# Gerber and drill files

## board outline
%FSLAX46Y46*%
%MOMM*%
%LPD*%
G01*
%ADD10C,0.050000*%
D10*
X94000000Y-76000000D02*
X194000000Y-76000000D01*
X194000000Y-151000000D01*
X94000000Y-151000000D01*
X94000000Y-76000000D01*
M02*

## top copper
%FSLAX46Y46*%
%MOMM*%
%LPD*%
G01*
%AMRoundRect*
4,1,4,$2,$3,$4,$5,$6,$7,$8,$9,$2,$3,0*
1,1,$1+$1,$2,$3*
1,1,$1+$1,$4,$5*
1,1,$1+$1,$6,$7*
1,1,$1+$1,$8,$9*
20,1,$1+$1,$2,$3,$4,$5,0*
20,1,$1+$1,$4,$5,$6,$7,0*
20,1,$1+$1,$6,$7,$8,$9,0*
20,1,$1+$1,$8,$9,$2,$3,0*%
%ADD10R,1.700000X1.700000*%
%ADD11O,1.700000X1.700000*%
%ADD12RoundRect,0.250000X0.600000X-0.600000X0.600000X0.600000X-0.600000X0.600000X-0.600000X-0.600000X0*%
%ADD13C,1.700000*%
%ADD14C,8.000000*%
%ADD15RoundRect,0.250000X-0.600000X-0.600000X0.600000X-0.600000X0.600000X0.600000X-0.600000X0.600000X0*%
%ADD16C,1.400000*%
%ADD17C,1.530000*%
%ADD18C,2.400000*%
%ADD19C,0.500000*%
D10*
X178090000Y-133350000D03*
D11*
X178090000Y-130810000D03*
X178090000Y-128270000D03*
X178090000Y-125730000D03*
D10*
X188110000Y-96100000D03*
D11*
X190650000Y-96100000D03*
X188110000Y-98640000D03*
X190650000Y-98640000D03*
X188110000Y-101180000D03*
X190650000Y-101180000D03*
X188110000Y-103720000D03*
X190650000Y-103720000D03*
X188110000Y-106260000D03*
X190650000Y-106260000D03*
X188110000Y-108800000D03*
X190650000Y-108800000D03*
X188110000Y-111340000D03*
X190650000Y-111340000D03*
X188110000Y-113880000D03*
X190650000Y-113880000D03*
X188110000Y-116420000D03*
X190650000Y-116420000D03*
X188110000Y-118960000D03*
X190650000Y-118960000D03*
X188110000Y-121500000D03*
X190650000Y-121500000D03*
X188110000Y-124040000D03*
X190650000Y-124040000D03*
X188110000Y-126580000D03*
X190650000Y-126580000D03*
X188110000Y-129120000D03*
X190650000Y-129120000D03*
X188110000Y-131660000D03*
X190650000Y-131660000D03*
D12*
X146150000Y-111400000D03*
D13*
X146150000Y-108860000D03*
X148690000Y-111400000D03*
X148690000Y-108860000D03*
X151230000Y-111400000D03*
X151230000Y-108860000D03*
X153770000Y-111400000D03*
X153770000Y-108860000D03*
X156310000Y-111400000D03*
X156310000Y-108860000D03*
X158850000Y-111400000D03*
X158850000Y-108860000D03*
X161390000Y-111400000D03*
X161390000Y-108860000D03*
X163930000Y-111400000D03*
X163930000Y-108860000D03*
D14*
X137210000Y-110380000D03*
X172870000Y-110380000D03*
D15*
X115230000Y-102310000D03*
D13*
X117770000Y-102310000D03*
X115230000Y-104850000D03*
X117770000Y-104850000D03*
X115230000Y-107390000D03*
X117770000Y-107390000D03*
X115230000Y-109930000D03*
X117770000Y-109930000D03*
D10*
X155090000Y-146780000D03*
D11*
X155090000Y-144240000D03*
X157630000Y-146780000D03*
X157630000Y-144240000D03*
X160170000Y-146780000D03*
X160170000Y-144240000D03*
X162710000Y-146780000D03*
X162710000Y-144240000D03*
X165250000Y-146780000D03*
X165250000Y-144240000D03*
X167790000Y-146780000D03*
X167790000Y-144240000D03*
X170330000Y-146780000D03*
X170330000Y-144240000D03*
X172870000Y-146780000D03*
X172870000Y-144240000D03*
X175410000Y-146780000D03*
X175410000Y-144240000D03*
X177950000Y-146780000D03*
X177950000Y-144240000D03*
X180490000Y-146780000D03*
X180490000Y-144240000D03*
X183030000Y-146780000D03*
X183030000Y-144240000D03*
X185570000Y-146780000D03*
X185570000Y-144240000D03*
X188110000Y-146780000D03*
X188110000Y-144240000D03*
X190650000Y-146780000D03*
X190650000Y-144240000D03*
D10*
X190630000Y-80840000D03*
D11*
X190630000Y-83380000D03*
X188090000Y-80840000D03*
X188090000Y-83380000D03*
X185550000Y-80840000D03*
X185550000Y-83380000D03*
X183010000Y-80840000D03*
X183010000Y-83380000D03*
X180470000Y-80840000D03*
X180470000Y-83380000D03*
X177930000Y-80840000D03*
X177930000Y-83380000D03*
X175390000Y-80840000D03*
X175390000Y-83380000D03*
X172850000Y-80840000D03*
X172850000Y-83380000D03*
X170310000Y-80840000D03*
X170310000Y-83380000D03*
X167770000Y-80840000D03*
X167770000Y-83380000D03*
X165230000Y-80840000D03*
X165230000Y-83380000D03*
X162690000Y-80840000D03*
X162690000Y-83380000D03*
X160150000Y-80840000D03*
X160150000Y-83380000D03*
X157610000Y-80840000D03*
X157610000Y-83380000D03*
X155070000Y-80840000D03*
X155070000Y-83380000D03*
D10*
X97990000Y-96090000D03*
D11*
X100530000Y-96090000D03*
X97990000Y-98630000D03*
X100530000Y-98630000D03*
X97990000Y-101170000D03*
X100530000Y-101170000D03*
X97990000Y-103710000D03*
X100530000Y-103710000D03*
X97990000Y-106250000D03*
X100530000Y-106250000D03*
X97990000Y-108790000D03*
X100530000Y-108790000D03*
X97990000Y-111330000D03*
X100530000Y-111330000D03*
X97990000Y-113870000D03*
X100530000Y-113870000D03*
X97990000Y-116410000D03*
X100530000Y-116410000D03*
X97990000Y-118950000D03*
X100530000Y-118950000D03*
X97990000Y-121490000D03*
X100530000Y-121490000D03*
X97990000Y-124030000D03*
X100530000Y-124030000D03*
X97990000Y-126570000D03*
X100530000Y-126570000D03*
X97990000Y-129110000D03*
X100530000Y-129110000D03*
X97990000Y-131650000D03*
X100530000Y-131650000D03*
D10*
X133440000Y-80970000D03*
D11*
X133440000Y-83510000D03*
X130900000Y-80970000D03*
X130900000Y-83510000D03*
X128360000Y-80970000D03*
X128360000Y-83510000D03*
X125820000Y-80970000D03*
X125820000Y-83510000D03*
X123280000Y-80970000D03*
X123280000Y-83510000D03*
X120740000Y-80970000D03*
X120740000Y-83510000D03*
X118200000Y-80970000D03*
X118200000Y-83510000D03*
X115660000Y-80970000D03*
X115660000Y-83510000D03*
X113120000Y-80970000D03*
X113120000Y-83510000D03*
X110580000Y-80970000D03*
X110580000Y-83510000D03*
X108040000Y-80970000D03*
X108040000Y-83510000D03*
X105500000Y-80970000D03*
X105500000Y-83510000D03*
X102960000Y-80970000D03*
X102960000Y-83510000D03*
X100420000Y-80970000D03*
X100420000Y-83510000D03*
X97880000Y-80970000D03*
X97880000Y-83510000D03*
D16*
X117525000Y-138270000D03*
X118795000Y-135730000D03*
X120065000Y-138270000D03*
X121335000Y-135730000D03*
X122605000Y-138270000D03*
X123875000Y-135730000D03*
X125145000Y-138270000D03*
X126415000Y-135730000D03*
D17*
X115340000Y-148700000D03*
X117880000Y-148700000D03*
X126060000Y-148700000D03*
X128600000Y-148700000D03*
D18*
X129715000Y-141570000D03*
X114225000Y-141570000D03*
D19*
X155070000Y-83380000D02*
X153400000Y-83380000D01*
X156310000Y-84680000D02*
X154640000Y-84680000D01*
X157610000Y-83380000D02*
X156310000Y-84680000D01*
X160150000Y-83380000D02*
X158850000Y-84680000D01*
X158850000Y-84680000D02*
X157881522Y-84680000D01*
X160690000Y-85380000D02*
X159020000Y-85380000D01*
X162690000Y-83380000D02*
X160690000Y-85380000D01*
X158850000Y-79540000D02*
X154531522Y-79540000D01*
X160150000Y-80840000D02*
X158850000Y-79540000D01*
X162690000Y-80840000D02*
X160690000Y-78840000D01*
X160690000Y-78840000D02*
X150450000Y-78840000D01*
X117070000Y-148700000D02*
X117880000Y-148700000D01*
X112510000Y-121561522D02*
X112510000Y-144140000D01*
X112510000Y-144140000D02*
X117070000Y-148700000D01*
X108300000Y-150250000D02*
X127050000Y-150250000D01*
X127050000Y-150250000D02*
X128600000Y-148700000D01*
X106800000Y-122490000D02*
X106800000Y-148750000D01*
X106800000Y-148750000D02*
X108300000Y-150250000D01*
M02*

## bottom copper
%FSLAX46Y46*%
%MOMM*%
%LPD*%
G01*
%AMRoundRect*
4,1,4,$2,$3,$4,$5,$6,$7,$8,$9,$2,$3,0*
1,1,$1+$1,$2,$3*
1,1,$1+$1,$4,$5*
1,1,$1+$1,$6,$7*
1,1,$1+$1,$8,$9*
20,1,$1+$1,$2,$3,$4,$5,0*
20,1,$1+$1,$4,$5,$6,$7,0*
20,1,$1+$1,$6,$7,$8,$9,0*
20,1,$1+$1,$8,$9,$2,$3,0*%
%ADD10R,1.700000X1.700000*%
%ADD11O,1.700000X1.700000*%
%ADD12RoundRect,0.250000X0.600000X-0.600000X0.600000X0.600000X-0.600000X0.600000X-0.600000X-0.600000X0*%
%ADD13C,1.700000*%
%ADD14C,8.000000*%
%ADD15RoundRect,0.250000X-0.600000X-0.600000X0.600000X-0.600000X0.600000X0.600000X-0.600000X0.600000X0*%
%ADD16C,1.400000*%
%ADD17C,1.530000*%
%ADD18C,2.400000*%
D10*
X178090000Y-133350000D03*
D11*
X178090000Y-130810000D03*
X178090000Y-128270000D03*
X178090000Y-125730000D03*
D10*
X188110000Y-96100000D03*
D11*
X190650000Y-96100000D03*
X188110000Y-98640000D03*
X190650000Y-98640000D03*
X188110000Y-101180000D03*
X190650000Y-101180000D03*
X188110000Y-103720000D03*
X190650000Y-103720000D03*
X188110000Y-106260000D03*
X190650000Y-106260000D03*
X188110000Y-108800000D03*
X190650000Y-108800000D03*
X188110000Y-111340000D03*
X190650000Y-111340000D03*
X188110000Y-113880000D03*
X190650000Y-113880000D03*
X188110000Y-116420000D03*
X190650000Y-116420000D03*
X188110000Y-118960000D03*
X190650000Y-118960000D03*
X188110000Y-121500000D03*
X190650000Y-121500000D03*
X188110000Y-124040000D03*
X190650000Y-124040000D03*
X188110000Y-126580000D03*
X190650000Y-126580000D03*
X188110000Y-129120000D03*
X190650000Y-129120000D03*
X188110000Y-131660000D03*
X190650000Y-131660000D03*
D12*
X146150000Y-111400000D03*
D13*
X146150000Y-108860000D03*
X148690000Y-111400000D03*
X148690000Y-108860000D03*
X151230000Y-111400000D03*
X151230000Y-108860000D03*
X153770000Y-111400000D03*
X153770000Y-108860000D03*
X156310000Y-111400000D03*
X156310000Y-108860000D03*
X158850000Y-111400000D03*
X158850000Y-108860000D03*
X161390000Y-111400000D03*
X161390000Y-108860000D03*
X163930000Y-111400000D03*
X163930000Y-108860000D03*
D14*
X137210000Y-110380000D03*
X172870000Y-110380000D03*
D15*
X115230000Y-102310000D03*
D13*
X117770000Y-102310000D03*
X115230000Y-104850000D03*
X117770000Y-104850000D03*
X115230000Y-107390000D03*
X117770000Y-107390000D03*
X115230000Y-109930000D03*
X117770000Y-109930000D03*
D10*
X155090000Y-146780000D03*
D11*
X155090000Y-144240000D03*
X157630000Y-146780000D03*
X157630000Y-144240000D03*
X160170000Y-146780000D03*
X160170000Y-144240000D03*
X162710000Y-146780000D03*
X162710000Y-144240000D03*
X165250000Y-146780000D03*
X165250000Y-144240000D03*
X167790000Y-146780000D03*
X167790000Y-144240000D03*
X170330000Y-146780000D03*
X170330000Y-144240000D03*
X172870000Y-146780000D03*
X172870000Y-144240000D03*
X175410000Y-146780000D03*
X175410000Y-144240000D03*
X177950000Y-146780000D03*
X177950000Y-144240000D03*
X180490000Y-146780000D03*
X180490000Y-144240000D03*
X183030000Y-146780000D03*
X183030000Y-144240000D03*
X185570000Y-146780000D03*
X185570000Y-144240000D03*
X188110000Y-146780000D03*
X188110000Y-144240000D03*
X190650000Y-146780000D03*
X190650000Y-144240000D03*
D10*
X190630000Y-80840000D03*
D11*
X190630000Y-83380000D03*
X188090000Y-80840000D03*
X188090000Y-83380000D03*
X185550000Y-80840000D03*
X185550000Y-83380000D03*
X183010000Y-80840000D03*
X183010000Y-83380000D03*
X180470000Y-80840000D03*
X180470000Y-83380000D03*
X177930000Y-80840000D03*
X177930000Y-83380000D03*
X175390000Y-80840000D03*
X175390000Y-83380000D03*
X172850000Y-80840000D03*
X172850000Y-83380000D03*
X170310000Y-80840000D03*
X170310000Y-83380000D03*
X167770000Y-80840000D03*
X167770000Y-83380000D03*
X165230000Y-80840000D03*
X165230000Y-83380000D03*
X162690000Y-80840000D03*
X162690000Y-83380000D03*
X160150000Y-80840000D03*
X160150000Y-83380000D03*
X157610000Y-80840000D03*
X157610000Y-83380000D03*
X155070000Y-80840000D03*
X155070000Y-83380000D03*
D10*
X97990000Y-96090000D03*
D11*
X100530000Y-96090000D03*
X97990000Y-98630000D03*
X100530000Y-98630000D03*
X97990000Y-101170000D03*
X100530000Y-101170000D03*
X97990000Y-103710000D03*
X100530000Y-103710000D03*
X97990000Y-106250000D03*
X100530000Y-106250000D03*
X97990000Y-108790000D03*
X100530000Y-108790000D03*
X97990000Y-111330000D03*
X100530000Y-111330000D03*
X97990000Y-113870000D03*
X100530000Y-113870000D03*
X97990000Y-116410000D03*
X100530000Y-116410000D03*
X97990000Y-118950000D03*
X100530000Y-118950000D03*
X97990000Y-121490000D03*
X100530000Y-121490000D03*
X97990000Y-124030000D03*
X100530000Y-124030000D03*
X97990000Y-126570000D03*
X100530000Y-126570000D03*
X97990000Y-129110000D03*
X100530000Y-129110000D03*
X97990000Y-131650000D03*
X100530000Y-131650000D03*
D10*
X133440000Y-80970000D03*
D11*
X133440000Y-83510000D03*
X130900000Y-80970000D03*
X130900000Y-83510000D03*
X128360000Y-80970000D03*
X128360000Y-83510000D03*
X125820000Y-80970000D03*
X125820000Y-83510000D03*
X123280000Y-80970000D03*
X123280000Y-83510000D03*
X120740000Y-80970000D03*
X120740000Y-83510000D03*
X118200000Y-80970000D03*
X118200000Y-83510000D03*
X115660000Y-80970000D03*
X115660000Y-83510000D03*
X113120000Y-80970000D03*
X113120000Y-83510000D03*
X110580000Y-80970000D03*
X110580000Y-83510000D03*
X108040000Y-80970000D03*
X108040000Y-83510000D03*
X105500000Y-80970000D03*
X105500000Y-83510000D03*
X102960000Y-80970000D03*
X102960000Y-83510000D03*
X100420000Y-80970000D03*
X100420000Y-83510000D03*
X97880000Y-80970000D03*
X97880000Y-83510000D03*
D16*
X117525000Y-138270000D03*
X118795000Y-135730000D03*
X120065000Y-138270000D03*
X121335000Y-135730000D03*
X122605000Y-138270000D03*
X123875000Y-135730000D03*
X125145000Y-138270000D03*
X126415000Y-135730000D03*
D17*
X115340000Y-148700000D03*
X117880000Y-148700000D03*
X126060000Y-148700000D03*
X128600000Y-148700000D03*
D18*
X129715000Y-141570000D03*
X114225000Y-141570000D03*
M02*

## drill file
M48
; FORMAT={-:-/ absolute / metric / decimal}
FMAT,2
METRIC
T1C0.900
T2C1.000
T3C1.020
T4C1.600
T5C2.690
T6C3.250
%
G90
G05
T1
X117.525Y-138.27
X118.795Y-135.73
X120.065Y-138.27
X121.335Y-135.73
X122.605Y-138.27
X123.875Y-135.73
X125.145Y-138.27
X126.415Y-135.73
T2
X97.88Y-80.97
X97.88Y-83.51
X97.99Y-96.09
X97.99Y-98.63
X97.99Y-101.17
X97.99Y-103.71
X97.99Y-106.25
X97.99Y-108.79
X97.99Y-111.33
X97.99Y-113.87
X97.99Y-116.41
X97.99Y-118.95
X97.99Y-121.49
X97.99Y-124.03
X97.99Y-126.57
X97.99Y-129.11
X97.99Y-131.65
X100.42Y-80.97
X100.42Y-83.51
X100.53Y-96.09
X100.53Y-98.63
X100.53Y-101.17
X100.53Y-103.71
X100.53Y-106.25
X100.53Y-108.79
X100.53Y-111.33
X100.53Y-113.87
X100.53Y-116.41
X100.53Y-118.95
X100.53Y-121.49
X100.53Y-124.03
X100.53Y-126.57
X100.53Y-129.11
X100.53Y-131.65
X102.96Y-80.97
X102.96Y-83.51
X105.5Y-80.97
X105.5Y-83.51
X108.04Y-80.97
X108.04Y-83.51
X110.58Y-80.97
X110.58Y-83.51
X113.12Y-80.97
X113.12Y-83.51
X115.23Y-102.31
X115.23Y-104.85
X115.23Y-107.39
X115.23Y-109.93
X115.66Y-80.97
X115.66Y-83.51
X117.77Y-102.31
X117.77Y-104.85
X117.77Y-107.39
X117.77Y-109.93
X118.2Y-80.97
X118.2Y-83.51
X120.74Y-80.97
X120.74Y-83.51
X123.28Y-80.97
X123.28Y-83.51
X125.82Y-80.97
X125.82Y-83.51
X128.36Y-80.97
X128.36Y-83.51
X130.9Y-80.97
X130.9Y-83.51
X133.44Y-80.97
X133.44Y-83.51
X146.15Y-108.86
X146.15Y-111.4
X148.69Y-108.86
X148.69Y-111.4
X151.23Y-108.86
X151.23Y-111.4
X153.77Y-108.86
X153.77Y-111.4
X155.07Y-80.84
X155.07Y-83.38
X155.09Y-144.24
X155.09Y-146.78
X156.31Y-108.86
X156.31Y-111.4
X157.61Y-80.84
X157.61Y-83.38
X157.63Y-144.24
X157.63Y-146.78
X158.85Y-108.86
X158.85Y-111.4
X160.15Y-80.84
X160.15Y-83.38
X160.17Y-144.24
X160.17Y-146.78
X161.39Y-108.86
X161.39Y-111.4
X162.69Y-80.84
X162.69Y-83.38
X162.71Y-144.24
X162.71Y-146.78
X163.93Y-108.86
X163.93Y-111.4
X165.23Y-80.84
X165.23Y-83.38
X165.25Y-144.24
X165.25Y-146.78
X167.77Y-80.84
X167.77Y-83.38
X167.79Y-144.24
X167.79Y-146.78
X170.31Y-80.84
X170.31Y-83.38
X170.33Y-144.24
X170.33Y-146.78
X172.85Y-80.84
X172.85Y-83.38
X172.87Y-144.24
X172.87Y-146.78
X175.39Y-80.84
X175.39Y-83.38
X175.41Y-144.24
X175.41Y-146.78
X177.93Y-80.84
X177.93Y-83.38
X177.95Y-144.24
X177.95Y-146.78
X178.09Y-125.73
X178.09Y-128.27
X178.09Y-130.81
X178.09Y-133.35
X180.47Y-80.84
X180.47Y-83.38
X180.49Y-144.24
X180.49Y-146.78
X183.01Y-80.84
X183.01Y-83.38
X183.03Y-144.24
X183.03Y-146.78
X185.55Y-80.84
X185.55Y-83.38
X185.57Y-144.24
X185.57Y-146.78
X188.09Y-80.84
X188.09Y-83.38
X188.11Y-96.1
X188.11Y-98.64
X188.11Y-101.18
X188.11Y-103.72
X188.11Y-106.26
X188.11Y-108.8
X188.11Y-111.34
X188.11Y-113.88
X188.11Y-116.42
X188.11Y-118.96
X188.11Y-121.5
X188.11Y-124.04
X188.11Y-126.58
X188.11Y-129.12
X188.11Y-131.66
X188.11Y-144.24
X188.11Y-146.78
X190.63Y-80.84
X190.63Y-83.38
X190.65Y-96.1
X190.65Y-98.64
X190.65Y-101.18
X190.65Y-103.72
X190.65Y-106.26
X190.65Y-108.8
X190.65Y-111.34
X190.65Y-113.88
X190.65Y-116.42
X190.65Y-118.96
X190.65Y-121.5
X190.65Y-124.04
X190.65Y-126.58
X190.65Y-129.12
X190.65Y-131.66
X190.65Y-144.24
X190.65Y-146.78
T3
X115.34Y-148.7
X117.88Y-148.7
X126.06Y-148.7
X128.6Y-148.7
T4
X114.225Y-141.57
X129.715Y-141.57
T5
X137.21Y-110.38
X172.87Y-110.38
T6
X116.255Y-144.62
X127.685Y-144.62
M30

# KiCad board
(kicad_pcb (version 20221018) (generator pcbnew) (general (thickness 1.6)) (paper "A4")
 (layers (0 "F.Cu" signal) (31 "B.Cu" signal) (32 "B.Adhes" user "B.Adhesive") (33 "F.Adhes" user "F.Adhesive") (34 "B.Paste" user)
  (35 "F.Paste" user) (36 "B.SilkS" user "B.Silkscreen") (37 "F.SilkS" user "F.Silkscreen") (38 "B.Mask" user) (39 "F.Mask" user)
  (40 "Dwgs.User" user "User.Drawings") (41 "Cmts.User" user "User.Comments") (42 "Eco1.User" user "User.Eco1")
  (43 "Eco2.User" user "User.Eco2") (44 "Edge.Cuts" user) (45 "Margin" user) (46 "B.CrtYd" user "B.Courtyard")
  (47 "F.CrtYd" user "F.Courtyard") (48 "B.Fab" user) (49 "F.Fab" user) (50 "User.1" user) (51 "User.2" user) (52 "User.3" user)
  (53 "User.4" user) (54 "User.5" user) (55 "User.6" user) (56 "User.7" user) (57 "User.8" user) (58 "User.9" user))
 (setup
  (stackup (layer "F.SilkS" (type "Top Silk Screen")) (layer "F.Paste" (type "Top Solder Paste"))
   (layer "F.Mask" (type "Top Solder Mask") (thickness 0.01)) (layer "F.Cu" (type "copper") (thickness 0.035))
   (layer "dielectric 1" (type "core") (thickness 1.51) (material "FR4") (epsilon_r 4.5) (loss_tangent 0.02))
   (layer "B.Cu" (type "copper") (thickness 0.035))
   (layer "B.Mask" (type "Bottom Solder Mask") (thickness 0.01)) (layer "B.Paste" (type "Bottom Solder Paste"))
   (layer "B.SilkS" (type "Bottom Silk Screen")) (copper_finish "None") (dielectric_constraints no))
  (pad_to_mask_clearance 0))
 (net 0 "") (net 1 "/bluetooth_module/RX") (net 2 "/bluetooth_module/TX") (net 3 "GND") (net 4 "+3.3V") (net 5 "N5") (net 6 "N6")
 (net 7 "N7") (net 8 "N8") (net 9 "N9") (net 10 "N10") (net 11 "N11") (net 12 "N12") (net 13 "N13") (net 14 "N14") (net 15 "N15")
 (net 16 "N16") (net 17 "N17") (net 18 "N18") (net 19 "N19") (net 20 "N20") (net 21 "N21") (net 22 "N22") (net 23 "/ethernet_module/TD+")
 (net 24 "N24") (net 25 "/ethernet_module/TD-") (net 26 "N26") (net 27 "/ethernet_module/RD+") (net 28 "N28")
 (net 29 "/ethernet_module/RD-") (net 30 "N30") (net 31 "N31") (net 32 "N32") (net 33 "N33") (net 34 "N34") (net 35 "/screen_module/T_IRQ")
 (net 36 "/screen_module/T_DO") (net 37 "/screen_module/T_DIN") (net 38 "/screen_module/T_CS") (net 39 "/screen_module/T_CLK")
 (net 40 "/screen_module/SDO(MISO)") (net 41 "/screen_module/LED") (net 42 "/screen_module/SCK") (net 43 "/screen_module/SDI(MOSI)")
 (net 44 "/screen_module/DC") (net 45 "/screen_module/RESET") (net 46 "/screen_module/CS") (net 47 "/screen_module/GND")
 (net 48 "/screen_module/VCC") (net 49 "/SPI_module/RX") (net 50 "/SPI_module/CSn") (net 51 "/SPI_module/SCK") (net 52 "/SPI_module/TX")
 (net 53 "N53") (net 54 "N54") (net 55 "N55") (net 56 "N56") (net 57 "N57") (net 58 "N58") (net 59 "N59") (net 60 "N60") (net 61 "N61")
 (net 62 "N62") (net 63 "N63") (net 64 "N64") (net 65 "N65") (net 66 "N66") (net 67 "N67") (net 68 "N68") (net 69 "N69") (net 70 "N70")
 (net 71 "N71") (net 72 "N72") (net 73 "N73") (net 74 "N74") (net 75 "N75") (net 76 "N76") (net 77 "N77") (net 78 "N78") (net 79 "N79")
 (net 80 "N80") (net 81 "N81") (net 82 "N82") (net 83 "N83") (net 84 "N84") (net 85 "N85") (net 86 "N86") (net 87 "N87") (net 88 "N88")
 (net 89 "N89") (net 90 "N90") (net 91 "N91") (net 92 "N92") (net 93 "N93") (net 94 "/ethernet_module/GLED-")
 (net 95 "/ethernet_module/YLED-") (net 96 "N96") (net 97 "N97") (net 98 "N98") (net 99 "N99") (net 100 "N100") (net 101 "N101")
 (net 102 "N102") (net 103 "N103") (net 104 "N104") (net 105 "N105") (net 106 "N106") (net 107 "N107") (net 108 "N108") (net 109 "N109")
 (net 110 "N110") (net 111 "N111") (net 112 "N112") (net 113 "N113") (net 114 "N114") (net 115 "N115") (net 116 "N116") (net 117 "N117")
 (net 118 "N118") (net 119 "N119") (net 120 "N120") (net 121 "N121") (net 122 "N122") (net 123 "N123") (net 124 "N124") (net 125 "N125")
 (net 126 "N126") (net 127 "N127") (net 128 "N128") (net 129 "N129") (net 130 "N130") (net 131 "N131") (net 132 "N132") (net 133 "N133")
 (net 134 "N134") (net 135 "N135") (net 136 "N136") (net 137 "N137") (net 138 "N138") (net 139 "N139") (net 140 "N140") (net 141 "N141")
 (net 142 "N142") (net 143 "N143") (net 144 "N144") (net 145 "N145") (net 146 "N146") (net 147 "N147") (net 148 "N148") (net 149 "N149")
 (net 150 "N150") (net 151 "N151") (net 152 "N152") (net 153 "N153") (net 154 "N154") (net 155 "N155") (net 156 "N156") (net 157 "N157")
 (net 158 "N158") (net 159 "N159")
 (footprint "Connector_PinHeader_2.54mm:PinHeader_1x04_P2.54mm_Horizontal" (layer "F.Cu") (at 178.09 133.35 180)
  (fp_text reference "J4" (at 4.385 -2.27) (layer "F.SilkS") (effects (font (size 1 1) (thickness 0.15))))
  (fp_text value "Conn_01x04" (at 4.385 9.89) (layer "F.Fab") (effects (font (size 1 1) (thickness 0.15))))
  (pad "1" thru_hole rect (at 0 0 180) (size 1.7 1.7) (drill 1) (layers "*.Cu" "*.Mask") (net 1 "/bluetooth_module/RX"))
  (pad "2" thru_hole oval (at 0 2.54 180) (size 1.7 1.7) (drill 1) (layers "*.Cu" "*.Mask") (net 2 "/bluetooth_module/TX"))
  (pad "3" thru_hole oval (at 0 5.08 180) (size 1.7 1.7) (drill 1) (layers "*.Cu" "*.Mask") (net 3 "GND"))
  (pad "4" thru_hole oval (at 0 7.62 180) (size 1.7 1.7) (drill 1) (layers "*.Cu" "*.Mask") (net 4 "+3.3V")))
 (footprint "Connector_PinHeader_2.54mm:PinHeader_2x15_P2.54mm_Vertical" (layer "F.Cu") (at 188.11 96.1)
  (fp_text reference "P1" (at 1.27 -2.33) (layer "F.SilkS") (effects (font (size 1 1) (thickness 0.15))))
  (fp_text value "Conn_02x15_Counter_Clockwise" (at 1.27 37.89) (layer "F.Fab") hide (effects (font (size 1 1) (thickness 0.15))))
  (pad "1" thru_hole rect (at 0 0) (size 1.7 1.7) (drill 1) (layers "*.Cu" "*.Mask") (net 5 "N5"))
  (pad "2" thru_hole oval (at 2.54 0) (size 1.7 1.7) (drill 1) (layers "*.Cu" "*.Mask") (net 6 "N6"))
  (pad "3" thru_hole oval (at 0 2.54) (size 1.7 1.7) (drill 1) (layers "*.Cu" "*.Mask") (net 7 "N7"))
  (pad "4" thru_hole oval (at 2.54 2.54) (size 1.7 1.7) (drill 1) (layers "*.Cu" "*.Mask") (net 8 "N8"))
  (pad "5" thru_hole oval (at 0 5.08) (size 1.7 1.7) (drill 1) (layers "*.Cu" "*.Mask") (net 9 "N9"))
  (pad "6" thru_hole oval (at 2.54 5.08) (size 1.7 1.7) (drill 1) (layers "*.Cu" "*.Mask") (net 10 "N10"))
  (pad "7" thru_hole oval (at 0 7.62) (size 1.7 1.7) (drill 1) (layers "*.Cu" "*.Mask") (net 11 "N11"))
  (pad "8" thru_hole oval (at 2.54 7.62) (size 1.7 1.7) (drill 1) (layers "*.Cu" "*.Mask") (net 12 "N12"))
  (pad "9" thru_hole oval (at 0 10.16) (size 1.7 1.7) (drill 1) (layers "*.Cu" "*.Mask") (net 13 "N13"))
  (pad "10" thru_hole oval (at 2.54 10.16) (size 1.7 1.7) (drill 1) (layers "*.Cu" "*.Mask") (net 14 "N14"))
  (pad "11" thru_hole oval (at 0 12.7) (size 1.7 1.7) (drill 1) (layers "*.Cu" "*.Mask") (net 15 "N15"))
  (pad "12" thru_hole oval (at 2.54 12.7) (size 1.7 1.7) (drill 1) (layers "*.Cu" "*.Mask") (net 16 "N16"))
  (pad "13" thru_hole oval (at 0 15.24) (size 1.7 1.7) (drill 1) (layers "*.Cu" "*.Mask") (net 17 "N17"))
  (pad "14" thru_hole oval (at 2.54 15.24) (size 1.7 1.7) (drill 1) (layers "*.Cu" "*.Mask") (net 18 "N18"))
  (pad "15" thru_hole oval (at 0 17.78) (size 1.7 1.7) (drill 1) (layers "*.Cu" "*.Mask") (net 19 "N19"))
  (pad "16" thru_hole oval (at 2.54 17.78) (size 1.7 1.7) (drill 1) (layers "*.Cu" "*.Mask") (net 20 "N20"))
  (pad "17" thru_hole oval (at 0 20.32) (size 1.7 1.7) (drill 1) (layers "*.Cu" "*.Mask") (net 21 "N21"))
  (pad "18" thru_hole oval (at 2.54 20.32) (size 1.7 1.7) (drill 1) (layers "*.Cu" "*.Mask") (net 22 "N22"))
  (pad "19" thru_hole oval (at 0 22.86) (size 1.7 1.7) (drill 1) (layers "*.Cu" "*.Mask") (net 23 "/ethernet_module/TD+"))
  (pad "20" thru_hole oval (at 2.54 22.86) (size 1.7 1.7) (drill 1) (layers "*.Cu" "*.Mask") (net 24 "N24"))
  (pad "21" thru_hole oval (at 0 25.4) (size 1.7 1.7) (drill 1) (layers "*.Cu" "*.Mask") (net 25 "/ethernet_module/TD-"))
  (pad "22" thru_hole oval (at 2.54 25.4) (size 1.7 1.7) (drill 1) (layers "*.Cu" "*.Mask") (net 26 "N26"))
  (pad "23" thru_hole oval (at 0 27.94) (size 1.7 1.7) (drill 1) (layers "*.Cu" "*.Mask") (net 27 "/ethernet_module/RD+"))
  (pad "24" thru_hole oval (at 2.54 27.94) (size 1.7 1.7) (drill 1) (layers "*.Cu" "*.Mask") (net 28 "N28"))
  (pad "25" thru_hole oval (at 0 30.48) (size 1.7 1.7) (drill 1) (layers "*.Cu" "*.Mask") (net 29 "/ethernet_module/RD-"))
  (pad "26" thru_hole oval (at 2.54 30.48) (size 1.7 1.7) (drill 1) (layers "*.Cu" "*.Mask") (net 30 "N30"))
  (pad "27" thru_hole oval (at 0 33.02) (size 1.7 1.7) (drill 1) (layers "*.Cu" "*.Mask") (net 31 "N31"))
  (pad "28" thru_hole oval (at 2.54 33.02) (size 1.7 1.7) (drill 1) (layers "*.Cu" "*.Mask") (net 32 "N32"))
  (pad "29" thru_hole oval (at 0 35.56) (size 1.7 1.7) (drill 1) (layers "*.Cu" "*.Mask") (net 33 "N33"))
  (pad "30" thru_hole oval (at 2.54 35.56) (size 1.7 1.7) (drill 1) (layers "*.Cu" "*.Mask") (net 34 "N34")))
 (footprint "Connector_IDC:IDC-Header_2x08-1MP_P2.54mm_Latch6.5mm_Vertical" (layer "F.Cu") (at 146.15 111.4 90)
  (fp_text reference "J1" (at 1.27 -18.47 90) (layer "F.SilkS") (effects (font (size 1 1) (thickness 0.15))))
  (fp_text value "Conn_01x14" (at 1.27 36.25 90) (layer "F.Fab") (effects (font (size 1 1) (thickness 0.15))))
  (pad "1" thru_hole roundrect (at 0 0 90) (size 1.7 1.7) (drill 1) (layers "*.Cu" "*.Mask") (roundrect_rratio 0.147059)
   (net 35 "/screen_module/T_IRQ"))
  (pad "2" thru_hole circle (at 2.54 0 90) (size 1.7 1.7) (drill 1) (layers "*.Cu" "*.Mask") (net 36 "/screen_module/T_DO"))
  (pad "3" thru_hole circle (at 0 2.54 90) (size 1.7 1.7) (drill 1) (layers "*.Cu" "*.Mask") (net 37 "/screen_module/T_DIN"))
  (pad "4" thru_hole circle (at 2.54 2.54 90) (size 1.7 1.7) (drill 1) (layers "*.Cu" "*.Mask") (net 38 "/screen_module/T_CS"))
  (pad "5" thru_hole circle (at 0 5.08 90) (size 1.7 1.7) (drill 1) (layers "*.Cu" "*.Mask") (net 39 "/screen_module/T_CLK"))
  (pad "6" thru_hole circle (at 2.54 5.08 90) (size 1.7 1.7) (drill 1) (layers "*.Cu" "*.Mask") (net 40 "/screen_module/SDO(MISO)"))
  (pad "7" thru_hole circle (at 0 7.62 90) (size 1.7 1.7) (drill 1) (layers "*.Cu" "*.Mask") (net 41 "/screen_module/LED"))
  (pad "8" thru_hole circle (at 2.54 7.62 90) (size 1.7 1.7) (drill 1) (layers "*.Cu" "*.Mask") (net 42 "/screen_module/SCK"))
  (pad "9" thru_hole circle (at 0 10.16 90) (size 1.7 1.7) (drill 1) (layers "*.Cu" "*.Mask") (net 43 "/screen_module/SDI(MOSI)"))
  (pad "10" thru_hole circle (at 2.54 10.16 90) (size 1.7 1.7) (drill 1) (layers "*.Cu" "*.Mask") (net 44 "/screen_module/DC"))
  (pad "11" thru_hole circle (at 0 12.7 90) (size 1.7 1.7) (drill 1) (layers "*.Cu" "*.Mask") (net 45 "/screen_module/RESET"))
  (pad "12" thru_hole circle (at 2.54 12.7 90) (size 1.7 1.7) (drill 1) (layers "*.Cu" "*.Mask") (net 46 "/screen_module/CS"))
  (pad "13" thru_hole circle (at 0 15.24 90) (size 1.7 1.7) (drill 1) (layers "*.Cu" "*.Mask") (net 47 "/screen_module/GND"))
  (pad "14" thru_hole circle (at 2.54 15.24 90) (size 1.7 1.7) (drill 1) (layers "*.Cu" "*.Mask") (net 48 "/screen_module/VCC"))
  (pad "15" thru_hole circle (at 0 17.78 90) (size 1.7 1.7) (drill 1) (layers "*.Cu" "*.Mask"))
  (pad "16" thru_hole circle (at 2.54 17.78 90) (size 1.7 1.7) (drill 1) (layers "*.Cu" "*.Mask"))
  (pad "MP" thru_hole circle (at 1.02 -8.94 90) (size 8 8) (drill 2.69) (layers "*.Cu" "*.Mask"))
  (pad "MP" thru_hole circle (at 1.02 26.72 90) (size 8 8) (drill 2.69) (layers "*.Cu" "*.Mask")))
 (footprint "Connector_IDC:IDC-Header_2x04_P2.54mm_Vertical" (layer "F.Cu") (at 115.23 102.31)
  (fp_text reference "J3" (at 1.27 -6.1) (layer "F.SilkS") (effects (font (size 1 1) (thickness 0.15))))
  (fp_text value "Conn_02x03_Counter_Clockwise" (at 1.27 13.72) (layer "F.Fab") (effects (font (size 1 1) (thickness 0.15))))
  (pad "1" thru_hole roundrect (at 0 0) (size 1.7 1.7) (drill 1) (layers "*.Cu" "*.Mask") (roundrect_rratio 0.147059) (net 3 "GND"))
  (pad "2" thru_hole circle (at 2.54 0) (size 1.7 1.7) (drill 1) (layers "*.Cu" "*.Mask") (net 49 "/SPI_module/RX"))
  (pad "3" thru_hole circle (at 0 2.54) (size 1.7 1.7) (drill 1) (layers "*.Cu" "*.Mask") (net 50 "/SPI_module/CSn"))
  (pad "4" thru_hole circle (at 2.54 2.54) (size 1.7 1.7) (drill 1) (layers "*.Cu" "*.Mask") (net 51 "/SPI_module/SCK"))
  (pad "5" thru_hole circle (at 0 5.08) (size 1.7 1.7) (drill 1) (layers "*.Cu" "*.Mask") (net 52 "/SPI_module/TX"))
  (pad "6" thru_hole circle (at 2.54 5.08) (size 1.7 1.7) (drill 1) (layers "*.Cu" "*.Mask") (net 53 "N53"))
  (pad "7" thru_hole circle (at 0 7.62) (size 1.7 1.7) (drill 1) (layers "*.Cu" "*.Mask"))
  (pad "8" thru_hole circle (at 2.54 7.62) (size 1.7 1.7) (drill 1) (layers "*.Cu" "*.Mask")))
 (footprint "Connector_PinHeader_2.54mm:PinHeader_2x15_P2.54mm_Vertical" (layer "F.Cu") (at 155.09 146.78 90)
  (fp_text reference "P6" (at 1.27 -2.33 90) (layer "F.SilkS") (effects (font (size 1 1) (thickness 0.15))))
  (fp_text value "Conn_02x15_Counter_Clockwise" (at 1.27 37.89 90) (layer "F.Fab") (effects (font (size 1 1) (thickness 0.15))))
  (pad "1" thru_hole rect (at 0 0 90) (size 1.7 1.7) (drill 1) (layers "*.Cu" "*.Mask") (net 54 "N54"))
  (pad "2" thru_hole oval (at 2.54 0 90) (size 1.7 1.7) (drill 1) (layers "*.Cu" "*.Mask") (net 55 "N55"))
  (pad "3" thru_hole oval (at 0 2.54 90) (size 1.7 1.7) (drill 1) (layers "*.Cu" "*.Mask") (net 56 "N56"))
  (pad "4" thru_hole oval (at 2.54 2.54 90) (size 1.7 1.7) (drill 1) (layers "*.Cu" "*.Mask") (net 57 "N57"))
  (pad "5" thru_hole oval (at 0 5.08 90) (size 1.7 1.7) (drill 1) (layers "*.Cu" "*.Mask") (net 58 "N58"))
  (pad "6" thru_hole oval (at 2.54 5.08 90) (size 1.7 1.7) (drill 1) (layers "*.Cu" "*.Mask") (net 1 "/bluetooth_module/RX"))
  (pad "7" thru_hole oval (at 0 7.62 90) (size 1.7 1.7) (drill 1) (layers "*.Cu" "*.Mask") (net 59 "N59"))
  (pad "8" thru_hole oval (at 2.54 7.62 90) (size 1.7 1.7) (drill 1) (layers "*.Cu" "*.Mask") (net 2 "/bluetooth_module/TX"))
  (pad "9" thru_hole oval (at 0 10.16 90) (size 1.7 1.7) (drill 1) (layers "*.Cu" "*.Mask") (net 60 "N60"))
  (pad "10" thru_hole oval (at 2.54 10.16 90) (size 1.7 1.7) (drill 1) (layers "*.Cu" "*.Mask") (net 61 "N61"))
  (pad "11" thru_hole oval (at 0 12.7 90) (size 1.7 1.7) (drill 1) (layers "*.Cu" "*.Mask") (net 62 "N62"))
  (pad "12" thru_hole oval (at 2.54 12.7 90) (size 1.7 1.7) (drill 1) (layers "*.Cu" "*.Mask") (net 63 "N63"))
  (pad "13" thru_hole oval (at 0 15.24 90) (size 1.7 1.7) (drill 1) (layers "*.Cu" "*.Mask") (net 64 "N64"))
  (pad "14" thru_hole oval (at 2.54 15.24 90) (size 1.7 1.7) (drill 1) (layers "*.Cu" "*.Mask") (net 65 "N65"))
  (pad "15" thru_hole oval (at 0 17.78 90) (size 1.7 1.7) (drill 1) (layers "*.Cu" "*.Mask") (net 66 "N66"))
  (pad "16" thru_hole oval (at 2.54 17.78 90) (size 1.7 1.7) (drill 1) (layers "*.Cu" "*.Mask") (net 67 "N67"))
  (pad "17" thru_hole oval (at 0 20.32 90) (size 1.7 1.7) (drill 1) (layers "*.Cu" "*.Mask") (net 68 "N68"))
  (pad "18" thru_hole oval (at 2.54 20.32 90) (size 1.7 1.7) (drill 1) (layers "*.Cu" "*.Mask") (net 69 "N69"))
  (pad "19" thru_hole oval (at 0 22.86 90) (size 1.7 1.7) (drill 1) (layers "*.Cu" "*.Mask") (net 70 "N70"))
  (pad "20" thru_hole oval (at 2.54 22.86 90) (size 1.7 1.7) (drill 1) (layers "*.Cu" "*.Mask") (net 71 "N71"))
  (pad "21" thru_hole oval (at 0 25.4 90) (size 1.7 1.7) (drill 1) (layers "*.Cu" "*.Mask") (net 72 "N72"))
  (pad "22" thru_hole oval (at 2.54 25.4 90) (size 1.7 1.7) (drill 1) (layers "*.Cu" "*.Mask") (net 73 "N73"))
  (pad "23" thru_hole oval (at 0 27.94 90) (size 1.7 1.7) (drill 1) (layers "*.Cu" "*.Mask") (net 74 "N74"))
  (pad "24" thru_hole oval (at 2.54 27.94 90) (size 1.7 1.7) (drill 1) (layers "*.Cu" "*.Mask") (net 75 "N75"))
  (pad "25" thru_hole oval (at 0 30.48 90) (size 1.7 1.7) (drill 1) (layers "*.Cu" "*.Mask") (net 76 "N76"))
  (pad "26" thru_hole oval (at 2.54 30.48 90) (size 1.7 1.7) (drill 1) (layers "*.Cu" "*.Mask") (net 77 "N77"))
  (pad "27" thru_hole oval (at 0 33.02 90) (size 1.7 1.7) (drill 1) (layers "*.Cu" "*.Mask") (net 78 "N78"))
  (pad "28" thru_hole oval (at 2.54 33.02 90) (size 1.7 1.7) (drill 1) (layers "*.Cu" "*.Mask") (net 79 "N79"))
  (pad "29" thru_hole oval (at 0 35.56 90) (size 1.7 1.7) (drill 1) (layers "*.Cu" "*.Mask") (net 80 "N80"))
  (pad "30" thru_hole oval (at 2.54 35.56 90) (size 1.7 1.7) (drill 1) (layers "*.Cu" "*.Mask") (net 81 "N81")))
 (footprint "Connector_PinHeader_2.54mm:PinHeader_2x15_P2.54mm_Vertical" (layer "F.Cu") (at 190.63 80.84 -90)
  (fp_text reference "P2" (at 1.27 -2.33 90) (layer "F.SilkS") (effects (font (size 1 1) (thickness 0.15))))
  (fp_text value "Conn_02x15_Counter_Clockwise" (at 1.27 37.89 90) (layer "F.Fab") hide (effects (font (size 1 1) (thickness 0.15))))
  (pad "1" thru_hole rect (at 0 0 270) (size 1.7 1.7) (drill 1) (layers "*.Cu" "*.Mask") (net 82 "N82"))
  (pad "2" thru_hole oval (at 2.54 0 270) (size 1.7 1.7) (drill 1) (layers "*.Cu" "*.Mask") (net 48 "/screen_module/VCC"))
  (pad "3" thru_hole oval (at 0 2.54 270) (size 1.7 1.7) (drill 1) (layers "*.Cu" "*.Mask") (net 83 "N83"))
  (pad "4" thru_hole oval (at 2.54 2.54 270) (size 1.7 1.7) (drill 1) (layers "*.Cu" "*.Mask") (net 47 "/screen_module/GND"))
  (pad "5" thru_hole oval (at 0 5.08 270) (size 1.7 1.7) (drill 1) (layers "*.Cu" "*.Mask") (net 42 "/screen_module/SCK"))
  (pad "6" thru_hole oval (at 2.54 5.08 270) (size 1.7 1.7) (drill 1) (layers "*.Cu" "*.Mask") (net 46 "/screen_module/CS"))
  (pad "7" thru_hole oval (at 0 7.62 270) (size 1.7 1.7) (drill 1) (layers "*.Cu" "*.Mask") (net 41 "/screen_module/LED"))
  (pad "8" thru_hole oval (at 2.54 7.62 270) (size 1.7 1.7) (drill 1) (layers "*.Cu" "*.Mask") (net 45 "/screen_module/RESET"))
  (pad "9" thru_hole oval (at 0 10.16 270) (size 1.7 1.7) (drill 1) (layers "*.Cu" "*.Mask") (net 40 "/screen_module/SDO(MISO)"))
  (pad "10" thru_hole oval (at 2.54 10.16 270) (size 1.7 1.7) (drill 1) (layers "*.Cu" "*.Mask") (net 44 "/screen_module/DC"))
  (pad "11" thru_hole oval (at 0 12.7 270) (size 1.7 1.7) (drill 1) (layers "*.Cu" "*.Mask") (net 39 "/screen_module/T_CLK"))
  (pad "12" thru_hole oval (at 2.54 12.7 270) (size 1.7 1.7) (drill 1) (layers "*.Cu" "*.Mask") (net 43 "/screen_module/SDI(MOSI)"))
  (pad "13" thru_hole oval (at 0 15.24 270) (size 1.7 1.7) (drill 1) (layers "*.Cu" "*.Mask") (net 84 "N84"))
  (pad "14" thru_hole oval (at 2.54 15.24 270) (size 1.7 1.7) (drill 1) (layers "*.Cu" "*.Mask") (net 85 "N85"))
  (pad "15" thru_hole oval (at 0 17.78 270) (size 1.7 1.7) (drill 1) (layers "*.Cu" "*.Mask") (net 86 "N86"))
  (pad "16" thru_hole oval (at 2.54 17.78 270) (size 1.7 1.7) (drill 1) (layers "*.Cu" "*.Mask") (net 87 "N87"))
  (pad "17" thru_hole oval (at 0 20.32 270) (size 1.7 1.7) (drill 1) (layers "*.Cu" "*.Mask") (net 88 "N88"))
  (pad "18" thru_hole oval (at 2.54 20.32 270) (size 1.7 1.7) (drill 1) (layers "*.Cu" "*.Mask") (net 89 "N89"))
  (pad "19" thru_hole oval (at 0 22.86 270) (size 1.7 1.7) (drill 1) (layers "*.Cu" "*.Mask") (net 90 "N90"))
  (pad "20" thru_hole oval (at 2.54 22.86 270) (size 1.7 1.7) (drill 1) (layers "*.Cu" "*.Mask") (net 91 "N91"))
  (pad "21" thru_hole oval (at 0 25.4 270) (size 1.7 1.7) (drill 1) (layers "*.Cu" "*.Mask") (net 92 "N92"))
  (pad "22" thru_hole oval (at 2.54 25.4 270) (size 1.7 1.7) (drill 1) (layers "*.Cu" "*.Mask") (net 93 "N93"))
  (pad "23" thru_hole oval (at 0 27.94 270) (size 1.7 1.7) (drill 1) (layers "*.Cu" "*.Mask") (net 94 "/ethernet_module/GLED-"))
  (pad "24" thru_hole oval (at 2.54 27.94 270) (size 1.7 1.7) (drill 1) (layers "*.Cu" "*.Mask") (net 38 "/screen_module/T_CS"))
  (pad "25" thru_hole oval (at 0 30.48 270) (size 1.7 1.7) (drill 1) (layers "*.Cu" "*.Mask") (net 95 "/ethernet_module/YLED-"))
  (pad "26" thru_hole oval (at 2.54 30.48 270) (size 1.7 1.7) (drill 1) (layers "*.Cu" "*.Mask") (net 37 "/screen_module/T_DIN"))
  (pad "27" thru_hole oval (at 0 33.02 270) (size 1.7 1.7) (drill 1) (layers "*.Cu" "*.Mask") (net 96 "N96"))
  (pad "28" thru_hole oval (at 2.54 33.02 270) (size 1.7 1.7) (drill 1) (layers "*.Cu" "*.Mask") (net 36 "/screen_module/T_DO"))
  (pad "29" thru_hole oval (at 0 35.56 270) (size 1.7 1.7) (drill 1) (layers "*.Cu" "*.Mask") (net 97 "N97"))
  (pad "30" thru_hole oval (at 2.54 35.56 270) (size 1.7 1.7) (drill 1) (layers "*.Cu" "*.Mask") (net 35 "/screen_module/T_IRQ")))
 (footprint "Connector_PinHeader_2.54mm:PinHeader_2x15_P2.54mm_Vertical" (layer "F.Cu") (at 97.99 96.09)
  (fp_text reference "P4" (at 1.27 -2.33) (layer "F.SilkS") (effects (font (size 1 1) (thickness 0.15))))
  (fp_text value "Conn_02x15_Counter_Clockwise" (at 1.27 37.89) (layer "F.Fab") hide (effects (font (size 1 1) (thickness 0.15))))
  (pad "1" thru_hole rect (at 0 0) (size 1.7 1.7) (drill 1) (layers "*.Cu" "*.Mask") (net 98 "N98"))
  (pad "2" thru_hole oval (at 2.54 0) (size 1.7 1.7) (drill 1) (layers "*.Cu" "*.Mask") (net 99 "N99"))
  (pad "3" thru_hole oval (at 0 2.54) (size 1.7 1.7) (drill 1) (layers "*.Cu" "*.Mask") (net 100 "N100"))
  (pad "4" thru_hole oval (at 2.54 2.54) (size 1.7 1.7) (drill 1) (layers "*.Cu" "*.Mask") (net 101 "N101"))
  (pad "5" thru_hole oval (at 0 5.08) (size 1.7 1.7) (drill 1) (layers "*.Cu" "*.Mask") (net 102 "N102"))
  (pad "6" thru_hole oval (at 2.54 5.08) (size 1.7 1.7) (drill 1) (layers "*.Cu" "*.Mask") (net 52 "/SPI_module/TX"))
  (pad "7" thru_hole oval (at 0 7.62) (size 1.7 1.7) (drill 1) (layers "*.Cu" "*.Mask") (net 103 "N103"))
  (pad "8" thru_hole oval (at 2.54 7.62) (size 1.7 1.7) (drill 1) (layers "*.Cu" "*.Mask") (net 51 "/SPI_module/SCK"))
  (pad "9" thru_hole oval (at 0 10.16) (size 1.7 1.7) (drill 1) (layers "*.Cu" "*.Mask") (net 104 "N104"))
  (pad "10" thru_hole oval (at 2.54 10.16) (size 1.7 1.7) (drill 1) (layers "*.Cu" "*.Mask") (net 49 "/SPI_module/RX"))
  (pad "11" thru_hole oval (at 0 12.7) (size 1.7 1.7) (drill 1) (layers "*.Cu" "*.Mask") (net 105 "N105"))
  (pad "12" thru_hole oval (at 2.54 12.7) (size 1.7 1.7) (drill 1) (layers "*.Cu" "*.Mask") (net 50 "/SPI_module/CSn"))
  (pad "13" thru_hole oval (at 0 15.24) (size 1.7 1.7) (drill 1) (layers "*.Cu" "*.Mask") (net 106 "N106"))
  (pad "14" thru_hole oval (at 2.54 15.24) (size 1.7 1.7) (drill 1) (layers "*.Cu" "*.Mask") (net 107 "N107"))
  (pad "15" thru_hole oval (at 0 17.78) (size 1.7 1.7) (drill 1) (layers "*.Cu" "*.Mask") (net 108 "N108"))
  (pad "16" thru_hole oval (at 2.54 17.78) (size 1.7 1.7) (drill 1) (layers "*.Cu" "*.Mask") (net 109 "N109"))
  (pad "17" thru_hole oval (at 0 20.32) (size 1.7 1.7) (drill 1) (layers "*.Cu" "*.Mask") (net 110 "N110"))
  (pad "18" thru_hole oval (at 2.54 20.32) (size 1.7 1.7) (drill 1) (layers "*.Cu" "*.Mask") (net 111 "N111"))
  (pad "19" thru_hole oval (at 0 22.86) (size 1.7 1.7) (drill 1) (layers "*.Cu" "*.Mask") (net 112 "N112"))
  (pad "20" thru_hole oval (at 2.54 22.86) (size 1.7 1.7) (drill 1) (layers "*.Cu" "*.Mask") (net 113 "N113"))
  (pad "21" thru_hole oval (at 0 25.4) (size 1.7 1.7) (drill 1) (layers "*.Cu" "*.Mask") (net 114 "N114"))
  (pad "22" thru_hole oval (at 2.54 25.4) (size 1.7 1.7) (drill 1) (layers "*.Cu" "*.Mask") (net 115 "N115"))
  (pad "23" thru_hole oval (at 0 27.94) (size 1.7 1.7) (drill 1) (layers "*.Cu" "*.Mask") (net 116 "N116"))
  (pad "24" thru_hole oval (at 2.54 27.94) (size 1.7 1.7) (drill 1) (layers "*.Cu" "*.Mask") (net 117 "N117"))
  (pad "25" thru_hole oval (at 0 30.48) (size 1.7 1.7) (drill 1) (layers "*.Cu" "*.Mask") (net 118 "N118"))
  (pad "26" thru_hole oval (at 2.54 30.48) (size 1.7 1.7) (drill 1) (layers "*.Cu" "*.Mask") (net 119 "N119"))
  (pad "27" thru_hole oval (at 0 33.02) (size 1.7 1.7) (drill 1) (layers "*.Cu" "*.Mask") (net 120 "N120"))
  (pad "28" thru_hole oval (at 2.54 33.02) (size 1.7 1.7) (drill 1) (layers "*.Cu" "*.Mask") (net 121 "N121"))
  (pad "29" thru_hole oval (at 0 35.56) (size 1.7 1.7) (drill 1) (layers "*.Cu" "*.Mask") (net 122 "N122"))
  (pad "30" thru_hole oval (at 2.54 35.56) (size 1.7 1.7) (drill 1) (layers "*.Cu" "*.Mask") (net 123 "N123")))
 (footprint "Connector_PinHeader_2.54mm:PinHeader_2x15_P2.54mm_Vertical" (layer "F.Cu") (at 133.44 80.97 -90)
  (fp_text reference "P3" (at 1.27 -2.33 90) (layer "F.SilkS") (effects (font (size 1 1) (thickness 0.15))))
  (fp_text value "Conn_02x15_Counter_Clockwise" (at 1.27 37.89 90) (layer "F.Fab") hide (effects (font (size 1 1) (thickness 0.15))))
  (pad "1" thru_hole rect (at 0 0 270) (size 1.7 1.7) (drill 1) (layers "*.Cu" "*.Mask") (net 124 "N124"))
  (pad "2" thru_hole oval (at 2.54 0 270) (size 1.7 1.7) (drill 1) (layers "*.Cu" "*.Mask") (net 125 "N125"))
  (pad "3" thru_hole oval (at 0 2.54 270) (size 1.7 1.7) (drill 1) (layers "*.Cu" "*.Mask") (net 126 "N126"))
  (pad "4" thru_hole oval (at 2.54 2.54 270) (size 1.7 1.7) (drill 1) (layers "*.Cu" "*.Mask") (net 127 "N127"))
  (pad "5" thru_hole oval (at 0 5.08 270) (size 1.7 1.7) (drill 1) (layers "*.Cu" "*.Mask") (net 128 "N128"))
  (pad "6" thru_hole oval (at 2.54 5.08 270) (size 1.7 1.7) (drill 1) (layers "*.Cu" "*.Mask") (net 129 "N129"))
  (pad "7" thru_hole oval (at 0 7.62 270) (size 1.7 1.7) (drill 1) (layers "*.Cu" "*.Mask") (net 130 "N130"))
  (pad "8" thru_hole oval (at 2.54 7.62 270) (size 1.7 1.7) (drill 1) (layers "*.Cu" "*.Mask") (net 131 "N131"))
  (pad "9" thru_hole oval (at 0 10.16 270) (size 1.7 1.7) (drill 1) (layers "*.Cu" "*.Mask") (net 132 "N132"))
  (pad "10" thru_hole oval (at 2.54 10.16 270) (size 1.7 1.7) (drill 1) (layers "*.Cu" "*.Mask") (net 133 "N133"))
  (pad "11" thru_hole oval (at 0 12.7 270) (size 1.7 1.7) (drill 1) (layers "*.Cu" "*.Mask") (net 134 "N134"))
  (pad "12" thru_hole oval (at 2.54 12.7 270) (size 1.7 1.7) (drill 1) (layers "*.Cu" "*.Mask") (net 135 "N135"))
  (pad "13" thru_hole oval (at 0 15.24 270) (size 1.7 1.7) (drill 1) (layers "*.Cu" "*.Mask") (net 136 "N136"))
  (pad "14" thru_hole oval (at 2.54 15.24 270) (size 1.7 1.7) (drill 1) (layers "*.Cu" "*.Mask") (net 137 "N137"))
  (pad "15" thru_hole oval (at 0 17.78 270) (size 1.7 1.7) (drill 1) (layers "*.Cu" "*.Mask") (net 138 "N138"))
  (pad "16" thru_hole oval (at 2.54 17.78 270) (size 1.7 1.7) (drill 1) (layers "*.Cu" "*.Mask") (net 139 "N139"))
  (pad "17" thru_hole oval (at 0 20.32 270) (size 1.7 1.7) (drill 1) (layers "*.Cu" "*.Mask") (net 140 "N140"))
  (pad "18" thru_hole oval (at 2.54 20.32 270) (size 1.7 1.7) (drill 1) (layers "*.Cu" "*.Mask") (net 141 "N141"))
  (pad "19" thru_hole oval (at 0 22.86 270) (size 1.7 1.7) (drill 1) (layers "*.Cu" "*.Mask") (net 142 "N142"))
  (pad "20" thru_hole oval (at 2.54 22.86 270) (size 1.7 1.7) (drill 1) (layers "*.Cu" "*.Mask") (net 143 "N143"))
  (pad "21" thru_hole oval (at 0 25.4 270) (size 1.7 1.7) (drill 1) (layers "*.Cu" "*.Mask") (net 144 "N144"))
  (pad "22" thru_hole oval (at 2.54 25.4 270) (size 1.7 1.7) (drill 1) (layers "*.Cu" "*.Mask") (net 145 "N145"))
  (pad "23" thru_hole oval (at 0 27.94 270) (size 1.7 1.7) (drill 1) (layers "*.Cu" "*.Mask") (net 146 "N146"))
  (pad "24" thru_hole oval (at 2.54 27.94 270) (size 1.7 1.7) (drill 1) (layers "*.Cu" "*.Mask") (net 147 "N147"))
  (pad "25" thru_hole oval (at 0 30.48 270) (size 1.7 1.7) (drill 1) (layers "*.Cu" "*.Mask") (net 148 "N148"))
  (pad "26" thru_hole oval (at 2.54 30.48 270) (size 1.7 1.7) (drill 1) (layers "*.Cu" "*.Mask") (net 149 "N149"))
  (pad "27" thru_hole oval (at 0 33.02 270) (size 1.7 1.7) (drill 1) (layers "*.Cu" "*.Mask") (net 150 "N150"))
  (pad "28" thru_hole oval (at 2.54 33.02 270) (size 1.7 1.7) (drill 1) (layers "*.Cu" "*.Mask") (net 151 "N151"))
  (pad "29" thru_hole oval (at 0 35.56 270) (size 1.7 1.7) (drill 1) (layers "*.Cu" "*.Mask") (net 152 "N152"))
  (pad "30" thru_hole oval (at 2.54 35.56 270) (size 1.7 1.7) (drill 1) (layers "*.Cu" "*.Mask") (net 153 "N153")))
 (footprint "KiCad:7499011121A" (layer "F.Cu") (at 121.97 144.59 180)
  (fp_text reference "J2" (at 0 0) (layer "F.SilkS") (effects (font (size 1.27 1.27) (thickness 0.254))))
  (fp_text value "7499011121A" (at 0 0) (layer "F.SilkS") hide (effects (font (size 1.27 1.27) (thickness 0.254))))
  (pad "" np_thru_hole circle (at -5.715 -0.03 180) (size 3.25 3.25) (drill 3.25) (layers "*.Cu" "*.Mask"))
  (pad "" np_thru_hole circle (at 5.715 -0.03 180) (size 3.25 3.25) (drill 3.25) (layers "*.Cu" "*.Mask"))
  (pad "1" thru_hole circle (at 4.445 6.32 180) (size 1.4 1.4) (drill 0.9) (layers "*.Cu" "*.Mask") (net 23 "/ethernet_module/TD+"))
  (pad "2" thru_hole circle (at 3.175 8.86 180) (size 1.4 1.4) (drill 0.9) (layers "*.Cu" "*.Mask") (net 4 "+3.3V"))
  (pad "3" thru_hole circle (at 1.905 6.32 180) (size 1.4 1.4) (drill 0.9) (layers "*.Cu" "*.Mask") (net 25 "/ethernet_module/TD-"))
  (pad "4" thru_hole circle (at 0.635 8.86 180) (size 1.4 1.4) (drill 0.9) (layers "*.Cu" "*.Mask") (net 27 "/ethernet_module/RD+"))
  (pad "5" thru_hole circle (at -0.635 6.32 180) (size 1.4 1.4) (drill 0.9) (layers "*.Cu" "*.Mask") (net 4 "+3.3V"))
  (pad "6" thru_hole circle (at -1.905 8.86 180) (size 1.4 1.4) (drill 0.9) (layers "*.Cu" "*.Mask") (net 29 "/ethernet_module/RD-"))
  (pad "7" thru_hole circle (at -3.175 6.32 180) (size 1.4 1.4) (drill 0.9) (layers "*.Cu" "*.Mask") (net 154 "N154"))
  (pad "8" thru_hole circle (at -4.445 8.86 180) (size 1.4 1.4) (drill 0.9) (layers "*.Cu" "*.Mask") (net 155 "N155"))
  (pad "9" thru_hole circle (at 6.63 -4.11 180) (size 1.53 1.53) (drill 1.02) (layers "*.Cu" "*.Mask") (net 4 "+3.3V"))
  (pad "10" thru_hole circle (at 4.09 -4.11 180) (size 1.53 1.53) (drill 1.02) (layers "*.Cu" "*.Mask") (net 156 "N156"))
  (pad "11" thru_hole circle (at -4.09 -4.11 180) (size 1.53 1.53) (drill 1.02) (layers "*.Cu" "*.Mask") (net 4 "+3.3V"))
  (pad "12" thru_hole circle (at -6.63 -4.11 180) (size 1.53 1.53) (drill 1.02) (layers "*.Cu" "*.Mask") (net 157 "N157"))
  (pad "13" thru_hole circle (at -7.745 3.02 180) (size 2.4 2.4) (drill 1.6) (layers "*.Cu" "*.Mask") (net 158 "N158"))
  (pad "14" thru_hole circle (at 7.745 3.02 180) (size 2.4 2.4) (drill 1.6) (layers "*.Cu" "*.Mask") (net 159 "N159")))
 (gr_rect (start 94 76) (end 194 151) (stroke (width 0.05) (type default)) (fill none) (layer "Edge.Cuts"))
 (segment (start 155.07 83.38) (end 153.4 83.38) (width 0.5) (layer "F.Cu") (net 35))
 (segment (start 156.31 84.68) (end 154.64 84.68) (width 0.5) (layer "F.Cu") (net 36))
 (segment (start 157.61 83.38) (end 156.31 84.68) (width 0.5) (layer "F.Cu") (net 36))
 (segment (start 160.15 83.38) (end 158.85 84.68) (width 0.5) (layer "F.Cu") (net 37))
 (segment (start 158.85 84.68) (end 157.881522 84.68) (width 0.5) (layer "F.Cu") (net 37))
 (segment (start 160.69 85.38) (end 159.02 85.38) (width 0.5) (layer "F.Cu") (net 38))
 (segment (start 162.69 83.38) (end 160.69 85.38) (width 0.5) (layer "F.Cu") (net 38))
 (segment (start 158.85 79.54) (end 154.531522 79.54) (width 0.5) (layer "F.Cu") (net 95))
 (segment (start 160.15 80.84) (end 158.85 79.54) (width 0.5) (layer "F.Cu") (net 95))
 (segment (start 162.69 80.84) (end 160.69 78.84) (width 0.5) (layer "F.Cu") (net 94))
 (segment (start 160.69 78.84) (end 150.45 78.84) (width 0.5) (layer "F.Cu") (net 94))
 (segment (start 117.07 148.7) (end 117.88 148.7) (width 0.5) (layer "F.Cu") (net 156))
 (segment (start 112.51 121.561522) (end 112.51 144.14) (width 0.5) (layer "F.Cu") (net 156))
 (segment (start 112.51 144.14) (end 117.07 148.7) (width 0.5) (layer "F.Cu") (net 156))
 (segment (start 108.3 150.25) (end 127.05 150.25) (width 0.5) (layer "F.Cu") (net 157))
 (segment (start 127.05 150.25) (end 128.6 148.7) (width 0.5) (layer "F.Cu") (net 157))
 (segment (start 106.8 122.49) (end 106.8 148.75) (width 0.5) (layer "F.Cu") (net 157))
 (segment (start 106.8 148.75) (end 108.3 150.25) (width 0.5) (layer "F.Cu") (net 157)))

